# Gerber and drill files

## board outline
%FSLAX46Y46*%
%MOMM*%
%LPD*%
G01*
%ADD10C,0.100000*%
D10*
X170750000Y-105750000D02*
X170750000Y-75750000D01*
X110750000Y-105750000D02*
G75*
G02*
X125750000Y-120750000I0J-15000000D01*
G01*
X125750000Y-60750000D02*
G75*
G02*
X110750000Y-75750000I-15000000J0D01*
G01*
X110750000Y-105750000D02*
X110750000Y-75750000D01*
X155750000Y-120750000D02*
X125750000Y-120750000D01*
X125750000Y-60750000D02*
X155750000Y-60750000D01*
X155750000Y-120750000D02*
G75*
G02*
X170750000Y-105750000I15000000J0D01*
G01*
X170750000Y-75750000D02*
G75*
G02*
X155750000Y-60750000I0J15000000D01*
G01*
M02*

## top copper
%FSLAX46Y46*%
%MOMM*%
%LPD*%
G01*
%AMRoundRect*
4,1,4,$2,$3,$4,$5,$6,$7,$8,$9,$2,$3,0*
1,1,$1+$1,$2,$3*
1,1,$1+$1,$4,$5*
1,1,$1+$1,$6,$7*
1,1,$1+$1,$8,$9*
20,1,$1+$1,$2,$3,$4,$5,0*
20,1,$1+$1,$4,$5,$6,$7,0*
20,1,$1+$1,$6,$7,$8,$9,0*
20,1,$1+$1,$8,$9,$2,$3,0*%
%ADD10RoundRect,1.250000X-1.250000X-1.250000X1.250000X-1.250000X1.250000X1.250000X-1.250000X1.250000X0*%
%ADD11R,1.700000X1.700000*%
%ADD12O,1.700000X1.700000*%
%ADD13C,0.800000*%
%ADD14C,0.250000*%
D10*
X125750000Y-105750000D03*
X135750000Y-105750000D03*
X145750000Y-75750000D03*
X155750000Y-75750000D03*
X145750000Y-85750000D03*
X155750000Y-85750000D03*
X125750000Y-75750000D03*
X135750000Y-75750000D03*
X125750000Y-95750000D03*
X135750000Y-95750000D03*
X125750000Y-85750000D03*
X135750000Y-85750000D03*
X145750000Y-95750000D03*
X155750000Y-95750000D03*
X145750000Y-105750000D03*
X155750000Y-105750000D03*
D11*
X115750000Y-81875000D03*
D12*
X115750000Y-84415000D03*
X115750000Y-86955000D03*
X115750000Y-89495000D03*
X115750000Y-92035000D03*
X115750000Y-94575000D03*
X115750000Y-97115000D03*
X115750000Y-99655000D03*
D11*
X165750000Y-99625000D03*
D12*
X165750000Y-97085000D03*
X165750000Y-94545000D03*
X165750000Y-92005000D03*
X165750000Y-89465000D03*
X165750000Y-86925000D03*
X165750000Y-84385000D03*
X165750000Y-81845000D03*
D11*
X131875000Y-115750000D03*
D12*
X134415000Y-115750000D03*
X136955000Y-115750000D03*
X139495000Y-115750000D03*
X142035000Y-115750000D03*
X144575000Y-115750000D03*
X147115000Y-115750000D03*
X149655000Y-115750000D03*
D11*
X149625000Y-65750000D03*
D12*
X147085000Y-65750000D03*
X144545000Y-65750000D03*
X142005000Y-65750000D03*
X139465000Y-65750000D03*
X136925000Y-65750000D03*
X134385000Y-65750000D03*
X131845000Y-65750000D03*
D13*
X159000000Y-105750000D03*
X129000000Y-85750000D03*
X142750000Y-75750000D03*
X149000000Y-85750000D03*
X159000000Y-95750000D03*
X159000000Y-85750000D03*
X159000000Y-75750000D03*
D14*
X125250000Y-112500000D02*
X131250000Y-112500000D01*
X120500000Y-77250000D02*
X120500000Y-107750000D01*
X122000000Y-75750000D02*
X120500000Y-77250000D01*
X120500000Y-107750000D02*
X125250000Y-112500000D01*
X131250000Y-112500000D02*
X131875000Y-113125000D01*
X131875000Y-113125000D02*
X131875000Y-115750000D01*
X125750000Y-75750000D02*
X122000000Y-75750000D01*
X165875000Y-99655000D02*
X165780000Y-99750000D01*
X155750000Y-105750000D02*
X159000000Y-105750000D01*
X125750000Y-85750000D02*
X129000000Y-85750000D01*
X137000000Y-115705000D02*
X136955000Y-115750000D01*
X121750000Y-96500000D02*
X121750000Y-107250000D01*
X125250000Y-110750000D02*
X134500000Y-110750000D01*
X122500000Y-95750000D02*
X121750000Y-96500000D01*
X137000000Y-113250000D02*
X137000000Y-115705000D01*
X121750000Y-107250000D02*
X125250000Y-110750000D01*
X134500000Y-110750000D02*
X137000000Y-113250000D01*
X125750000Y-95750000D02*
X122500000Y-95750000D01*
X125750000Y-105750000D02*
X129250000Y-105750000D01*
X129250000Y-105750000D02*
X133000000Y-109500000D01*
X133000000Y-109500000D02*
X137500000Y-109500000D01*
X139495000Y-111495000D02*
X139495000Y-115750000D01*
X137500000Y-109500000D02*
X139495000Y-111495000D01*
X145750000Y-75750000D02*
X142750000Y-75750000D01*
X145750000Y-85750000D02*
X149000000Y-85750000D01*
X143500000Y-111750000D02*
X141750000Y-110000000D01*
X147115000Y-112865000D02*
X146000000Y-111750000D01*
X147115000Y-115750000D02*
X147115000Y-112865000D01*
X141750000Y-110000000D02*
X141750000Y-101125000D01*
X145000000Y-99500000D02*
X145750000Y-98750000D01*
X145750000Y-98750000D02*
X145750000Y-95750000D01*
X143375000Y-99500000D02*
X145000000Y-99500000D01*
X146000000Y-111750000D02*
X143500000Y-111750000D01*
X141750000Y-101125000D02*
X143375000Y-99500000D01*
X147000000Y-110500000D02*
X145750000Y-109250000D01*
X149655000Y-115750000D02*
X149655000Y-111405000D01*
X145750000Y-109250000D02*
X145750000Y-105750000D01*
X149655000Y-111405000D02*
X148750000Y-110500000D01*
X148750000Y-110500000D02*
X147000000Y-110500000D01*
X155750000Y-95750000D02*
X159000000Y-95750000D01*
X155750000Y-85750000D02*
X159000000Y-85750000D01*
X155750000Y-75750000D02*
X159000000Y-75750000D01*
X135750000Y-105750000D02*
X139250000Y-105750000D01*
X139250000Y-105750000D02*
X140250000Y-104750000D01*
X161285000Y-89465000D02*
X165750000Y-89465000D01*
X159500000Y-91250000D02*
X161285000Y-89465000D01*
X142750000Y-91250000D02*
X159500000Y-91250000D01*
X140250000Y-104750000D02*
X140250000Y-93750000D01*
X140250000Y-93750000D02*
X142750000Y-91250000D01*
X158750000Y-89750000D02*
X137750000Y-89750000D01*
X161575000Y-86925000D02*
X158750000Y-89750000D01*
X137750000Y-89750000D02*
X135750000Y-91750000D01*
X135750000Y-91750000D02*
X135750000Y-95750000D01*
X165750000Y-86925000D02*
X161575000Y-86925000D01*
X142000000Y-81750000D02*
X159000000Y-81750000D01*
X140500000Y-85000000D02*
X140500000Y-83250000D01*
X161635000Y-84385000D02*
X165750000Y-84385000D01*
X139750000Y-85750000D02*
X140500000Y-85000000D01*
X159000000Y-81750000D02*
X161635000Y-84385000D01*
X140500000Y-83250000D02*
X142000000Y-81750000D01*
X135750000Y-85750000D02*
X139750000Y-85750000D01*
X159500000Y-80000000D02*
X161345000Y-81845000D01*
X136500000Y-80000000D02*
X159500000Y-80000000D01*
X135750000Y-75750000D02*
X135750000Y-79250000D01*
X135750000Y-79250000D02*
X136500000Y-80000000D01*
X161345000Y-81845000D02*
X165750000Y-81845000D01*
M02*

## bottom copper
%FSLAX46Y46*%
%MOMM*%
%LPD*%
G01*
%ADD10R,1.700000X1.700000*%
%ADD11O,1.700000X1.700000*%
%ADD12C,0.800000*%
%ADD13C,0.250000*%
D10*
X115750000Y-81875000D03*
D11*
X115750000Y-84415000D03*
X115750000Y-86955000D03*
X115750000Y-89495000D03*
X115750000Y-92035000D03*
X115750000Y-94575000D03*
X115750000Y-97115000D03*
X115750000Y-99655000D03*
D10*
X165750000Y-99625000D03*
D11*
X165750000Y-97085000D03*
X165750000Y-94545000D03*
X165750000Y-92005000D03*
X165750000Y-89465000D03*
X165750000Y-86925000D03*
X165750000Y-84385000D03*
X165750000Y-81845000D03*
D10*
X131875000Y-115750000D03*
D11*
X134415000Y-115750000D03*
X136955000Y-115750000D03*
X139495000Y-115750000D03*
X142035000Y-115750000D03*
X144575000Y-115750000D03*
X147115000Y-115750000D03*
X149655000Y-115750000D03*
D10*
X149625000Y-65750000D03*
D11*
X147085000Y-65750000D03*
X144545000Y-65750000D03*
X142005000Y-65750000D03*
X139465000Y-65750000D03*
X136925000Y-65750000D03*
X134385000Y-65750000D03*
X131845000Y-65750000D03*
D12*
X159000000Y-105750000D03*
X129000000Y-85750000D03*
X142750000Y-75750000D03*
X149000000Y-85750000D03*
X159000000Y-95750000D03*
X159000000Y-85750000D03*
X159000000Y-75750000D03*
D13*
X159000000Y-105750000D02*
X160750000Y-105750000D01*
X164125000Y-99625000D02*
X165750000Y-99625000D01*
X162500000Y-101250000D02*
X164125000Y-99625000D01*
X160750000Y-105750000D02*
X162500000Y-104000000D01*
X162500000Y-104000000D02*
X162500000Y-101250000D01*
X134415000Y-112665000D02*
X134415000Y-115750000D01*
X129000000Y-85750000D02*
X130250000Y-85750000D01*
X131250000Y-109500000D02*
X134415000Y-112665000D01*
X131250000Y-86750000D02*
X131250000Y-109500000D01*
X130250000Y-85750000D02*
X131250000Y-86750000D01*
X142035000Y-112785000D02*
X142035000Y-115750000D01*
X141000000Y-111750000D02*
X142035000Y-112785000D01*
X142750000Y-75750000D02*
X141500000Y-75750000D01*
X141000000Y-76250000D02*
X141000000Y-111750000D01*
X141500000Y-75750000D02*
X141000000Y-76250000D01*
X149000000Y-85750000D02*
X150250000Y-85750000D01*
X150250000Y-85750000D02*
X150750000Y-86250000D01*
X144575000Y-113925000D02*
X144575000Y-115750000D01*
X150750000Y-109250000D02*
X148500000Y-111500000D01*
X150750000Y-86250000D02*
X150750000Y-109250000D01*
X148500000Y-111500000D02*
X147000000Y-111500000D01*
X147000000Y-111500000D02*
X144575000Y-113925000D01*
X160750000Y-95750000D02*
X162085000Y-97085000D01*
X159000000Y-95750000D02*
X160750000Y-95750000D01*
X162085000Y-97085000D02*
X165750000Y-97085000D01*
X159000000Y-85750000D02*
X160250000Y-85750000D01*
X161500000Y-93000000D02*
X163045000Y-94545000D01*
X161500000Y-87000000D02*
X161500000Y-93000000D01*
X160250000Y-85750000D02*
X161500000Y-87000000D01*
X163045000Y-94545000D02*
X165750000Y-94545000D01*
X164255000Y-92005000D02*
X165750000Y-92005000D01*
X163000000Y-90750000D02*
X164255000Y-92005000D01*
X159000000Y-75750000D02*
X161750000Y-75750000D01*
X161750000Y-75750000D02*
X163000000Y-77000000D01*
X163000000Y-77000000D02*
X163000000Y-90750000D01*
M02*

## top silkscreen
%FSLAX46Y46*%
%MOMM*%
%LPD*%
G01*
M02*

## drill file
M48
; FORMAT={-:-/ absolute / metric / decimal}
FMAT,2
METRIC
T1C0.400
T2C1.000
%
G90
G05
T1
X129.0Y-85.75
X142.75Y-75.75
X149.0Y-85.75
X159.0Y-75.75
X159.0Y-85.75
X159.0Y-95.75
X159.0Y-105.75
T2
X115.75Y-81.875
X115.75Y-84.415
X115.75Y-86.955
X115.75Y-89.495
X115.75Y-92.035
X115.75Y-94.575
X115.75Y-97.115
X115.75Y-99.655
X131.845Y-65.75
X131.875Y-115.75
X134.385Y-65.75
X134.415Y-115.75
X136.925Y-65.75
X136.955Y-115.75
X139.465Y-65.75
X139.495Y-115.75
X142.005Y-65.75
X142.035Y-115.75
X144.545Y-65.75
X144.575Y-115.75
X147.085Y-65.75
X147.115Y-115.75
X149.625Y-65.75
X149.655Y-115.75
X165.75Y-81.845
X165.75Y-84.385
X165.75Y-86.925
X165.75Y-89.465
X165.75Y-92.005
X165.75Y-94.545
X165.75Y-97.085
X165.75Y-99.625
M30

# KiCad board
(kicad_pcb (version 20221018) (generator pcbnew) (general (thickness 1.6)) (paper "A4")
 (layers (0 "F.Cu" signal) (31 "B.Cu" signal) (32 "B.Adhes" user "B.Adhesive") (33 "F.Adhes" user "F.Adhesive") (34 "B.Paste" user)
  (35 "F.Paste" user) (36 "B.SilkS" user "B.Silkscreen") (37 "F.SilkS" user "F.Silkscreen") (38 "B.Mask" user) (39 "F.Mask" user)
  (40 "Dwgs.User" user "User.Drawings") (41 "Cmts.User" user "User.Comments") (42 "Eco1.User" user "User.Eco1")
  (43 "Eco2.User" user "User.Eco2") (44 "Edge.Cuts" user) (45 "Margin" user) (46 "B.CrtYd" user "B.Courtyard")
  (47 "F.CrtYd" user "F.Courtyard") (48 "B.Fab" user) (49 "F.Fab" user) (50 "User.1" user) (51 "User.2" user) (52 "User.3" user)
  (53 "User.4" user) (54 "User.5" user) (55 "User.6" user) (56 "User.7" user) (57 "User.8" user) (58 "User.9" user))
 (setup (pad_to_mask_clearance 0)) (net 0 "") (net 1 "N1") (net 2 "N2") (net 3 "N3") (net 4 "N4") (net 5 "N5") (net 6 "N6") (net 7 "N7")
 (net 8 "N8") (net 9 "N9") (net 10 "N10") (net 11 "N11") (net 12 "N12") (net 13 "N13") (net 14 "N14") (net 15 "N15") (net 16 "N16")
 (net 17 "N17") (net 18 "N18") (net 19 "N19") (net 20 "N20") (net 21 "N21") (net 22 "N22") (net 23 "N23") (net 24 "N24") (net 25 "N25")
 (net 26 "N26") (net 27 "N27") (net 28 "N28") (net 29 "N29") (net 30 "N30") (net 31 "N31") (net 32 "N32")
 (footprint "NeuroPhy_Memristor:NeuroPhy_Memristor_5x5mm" (layer "F.Cu") (at 130.75 105.75)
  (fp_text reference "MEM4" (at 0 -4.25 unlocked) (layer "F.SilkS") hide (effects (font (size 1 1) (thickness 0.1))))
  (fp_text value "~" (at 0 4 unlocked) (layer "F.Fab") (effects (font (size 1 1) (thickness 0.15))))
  (pad "1" smd roundrect (at -5 0) (size 5 5) (layers "F.Cu" "F.Mask") (roundrect_rratio 0.25) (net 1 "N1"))
  (pad "2" smd roundrect (at 5 0) (size 5 5) (layers "F.Cu" "F.Mask") (roundrect_rratio 0.25) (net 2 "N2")))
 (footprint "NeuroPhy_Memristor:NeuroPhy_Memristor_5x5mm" (layer "F.Cu") (at 150.75 75.75)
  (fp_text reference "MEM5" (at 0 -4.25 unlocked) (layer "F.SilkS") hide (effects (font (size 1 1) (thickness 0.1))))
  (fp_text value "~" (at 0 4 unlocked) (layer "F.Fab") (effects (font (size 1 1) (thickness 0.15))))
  (pad "1" smd roundrect (at -5 0) (size 5 5) (layers "F.Cu" "F.Mask") (roundrect_rratio 0.25) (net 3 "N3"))
  (pad "2" smd roundrect (at 5 0) (size 5 5) (layers "F.Cu" "F.Mask") (roundrect_rratio 0.25) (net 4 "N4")))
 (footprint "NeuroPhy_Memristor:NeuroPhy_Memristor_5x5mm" (layer "F.Cu") (at 150.75 85.75)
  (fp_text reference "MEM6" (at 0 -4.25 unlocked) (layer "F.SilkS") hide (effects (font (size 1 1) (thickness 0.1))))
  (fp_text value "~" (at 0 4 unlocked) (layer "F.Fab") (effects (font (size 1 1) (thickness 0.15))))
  (pad "1" smd roundrect (at -5 0) (size 5 5) (layers "F.Cu" "F.Mask") (roundrect_rratio 0.25) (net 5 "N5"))
  (pad "2" smd roundrect (at 5 0) (size 5 5) (layers "F.Cu" "F.Mask") (roundrect_rratio 0.25) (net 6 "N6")))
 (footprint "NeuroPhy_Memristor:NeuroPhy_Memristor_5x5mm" (layer "F.Cu") (at 130.75 75.75)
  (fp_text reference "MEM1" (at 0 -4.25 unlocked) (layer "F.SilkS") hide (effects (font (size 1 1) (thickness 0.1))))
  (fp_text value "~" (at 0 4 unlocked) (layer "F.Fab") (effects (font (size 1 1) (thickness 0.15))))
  (pad "1" smd roundrect (at -5 0) (size 5 5) (layers "F.Cu" "F.Mask") (roundrect_rratio 0.25) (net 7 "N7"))
  (pad "2" smd roundrect (at 5 0) (size 5 5) (layers "F.Cu" "F.Mask") (roundrect_rratio 0.25) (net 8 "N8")))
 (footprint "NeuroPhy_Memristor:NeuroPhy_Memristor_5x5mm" (layer "F.Cu") (at 130.75 95.75)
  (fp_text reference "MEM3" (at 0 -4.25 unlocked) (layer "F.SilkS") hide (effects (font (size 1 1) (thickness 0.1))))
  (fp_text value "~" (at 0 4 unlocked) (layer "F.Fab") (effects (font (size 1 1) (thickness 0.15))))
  (pad "1" smd roundrect (at -5 0) (size 5 5) (layers "F.Cu" "F.Mask") (roundrect_rratio 0.25) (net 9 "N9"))
  (pad "2" smd roundrect (at 5 0) (size 5 5) (layers "F.Cu" "F.Mask") (roundrect_rratio 0.25) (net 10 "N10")))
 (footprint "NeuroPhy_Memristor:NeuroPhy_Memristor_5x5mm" (layer "F.Cu") (at 130.75 85.75)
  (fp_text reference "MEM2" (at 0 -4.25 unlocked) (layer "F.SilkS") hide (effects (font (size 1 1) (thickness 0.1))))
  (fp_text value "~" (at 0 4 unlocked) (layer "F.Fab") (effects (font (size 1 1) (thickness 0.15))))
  (pad "1" smd roundrect (at -5 0) (size 5 5) (layers "F.Cu" "F.Mask") (roundrect_rratio 0.25) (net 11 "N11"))
  (pad "2" smd roundrect (at 5 0) (size 5 5) (layers "F.Cu" "F.Mask") (roundrect_rratio 0.25) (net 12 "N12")))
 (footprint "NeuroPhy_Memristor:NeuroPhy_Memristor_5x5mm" (layer "F.Cu") (at 150.75 95.75)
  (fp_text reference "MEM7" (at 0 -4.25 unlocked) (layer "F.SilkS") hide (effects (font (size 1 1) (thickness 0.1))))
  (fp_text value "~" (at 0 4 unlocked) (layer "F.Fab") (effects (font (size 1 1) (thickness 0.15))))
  (pad "1" smd roundrect (at -5 0) (size 5 5) (layers "F.Cu" "F.Mask") (roundrect_rratio 0.25) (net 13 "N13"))
  (pad "2" smd roundrect (at 5 0) (size 5 5) (layers "F.Cu" "F.Mask") (roundrect_rratio 0.25) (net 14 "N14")))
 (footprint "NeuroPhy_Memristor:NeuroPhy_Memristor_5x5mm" (layer "F.Cu") (at 150.75 105.75)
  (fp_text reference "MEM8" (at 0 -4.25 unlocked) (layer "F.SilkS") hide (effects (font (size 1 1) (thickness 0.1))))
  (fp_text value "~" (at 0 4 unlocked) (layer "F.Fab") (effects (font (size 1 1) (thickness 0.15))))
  (pad "1" smd roundrect (at -5 0) (size 5 5) (layers "F.Cu" "F.Mask") (roundrect_rratio 0.25) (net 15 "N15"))
  (pad "2" smd roundrect (at 5 0) (size 5 5) (layers "F.Cu" "F.Mask") (roundrect_rratio 0.25) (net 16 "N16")))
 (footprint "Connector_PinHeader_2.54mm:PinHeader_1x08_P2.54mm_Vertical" (layer "B.Cu") (at 115.75 81.875 180)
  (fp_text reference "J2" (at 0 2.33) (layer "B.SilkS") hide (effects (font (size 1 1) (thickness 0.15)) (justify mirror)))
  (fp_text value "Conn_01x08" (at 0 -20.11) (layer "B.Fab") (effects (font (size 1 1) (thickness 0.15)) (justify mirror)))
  (pad "1" thru_hole rect (at 0 0 180) (size 1.7 1.7) (drill 1) (layers "*.Cu" "*.Mask") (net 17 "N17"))
  (pad "2" thru_hole oval (at 0 -2.54 180) (size 1.7 1.7) (drill 1) (layers "*.Cu" "*.Mask") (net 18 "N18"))
  (pad "3" thru_hole oval (at 0 -5.08 180) (size 1.7 1.7) (drill 1) (layers "*.Cu" "*.Mask") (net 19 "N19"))
  (pad "4" thru_hole oval (at 0 -7.62 180) (size 1.7 1.7) (drill 1) (layers "*.Cu" "*.Mask") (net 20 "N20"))
  (pad "5" thru_hole oval (at 0 -10.16 180) (size 1.7 1.7) (drill 1) (layers "*.Cu" "*.Mask") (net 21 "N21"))
  (pad "6" thru_hole oval (at 0 -12.7 180) (size 1.7 1.7) (drill 1) (layers "*.Cu" "*.Mask") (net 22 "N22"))
  (pad "7" thru_hole oval (at 0 -15.24 180) (size 1.7 1.7) (drill 1) (layers "*.Cu" "*.Mask") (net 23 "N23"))
  (pad "8" thru_hole oval (at 0 -17.78 180) (size 1.7 1.7) (drill 1) (layers "*.Cu" "*.Mask") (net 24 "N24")))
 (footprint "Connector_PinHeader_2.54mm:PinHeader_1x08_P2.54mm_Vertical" (layer "B.Cu") (at 165.75 99.625)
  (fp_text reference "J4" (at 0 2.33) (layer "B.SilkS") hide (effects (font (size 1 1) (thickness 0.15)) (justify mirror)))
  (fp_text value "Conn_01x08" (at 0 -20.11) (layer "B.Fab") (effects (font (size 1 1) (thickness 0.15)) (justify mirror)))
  (pad "1" thru_hole rect (at 0 0) (size 1.7 1.7) (drill 1) (layers "*.Cu" "*.Mask") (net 16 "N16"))
  (pad "2" thru_hole oval (at 0 -2.54) (size 1.7 1.7) (drill 1) (layers "*.Cu" "*.Mask") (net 14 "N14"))
  (pad "3" thru_hole oval (at 0 -5.08) (size 1.7 1.7) (drill 1) (layers "*.Cu" "*.Mask") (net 6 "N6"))
  (pad "4" thru_hole oval (at 0 -7.62) (size 1.7 1.7) (drill 1) (layers "*.Cu" "*.Mask") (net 4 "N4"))
  (pad "5" thru_hole oval (at 0 -10.16) (size 1.7 1.7) (drill 1) (layers "*.Cu" "*.Mask") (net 2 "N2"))
  (pad "6" thru_hole oval (at 0 -12.7) (size 1.7 1.7) (drill 1) (layers "*.Cu" "*.Mask") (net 10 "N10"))
  (pad "7" thru_hole oval (at 0 -15.24) (size 1.7 1.7) (drill 1) (layers "*.Cu" "*.Mask") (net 12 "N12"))
  (pad "8" thru_hole oval (at 0 -17.78) (size 1.7 1.7) (drill 1) (layers "*.Cu" "*.Mask") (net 8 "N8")))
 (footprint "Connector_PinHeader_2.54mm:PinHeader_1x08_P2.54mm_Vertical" (layer "B.Cu") (at 131.875 115.75 -90)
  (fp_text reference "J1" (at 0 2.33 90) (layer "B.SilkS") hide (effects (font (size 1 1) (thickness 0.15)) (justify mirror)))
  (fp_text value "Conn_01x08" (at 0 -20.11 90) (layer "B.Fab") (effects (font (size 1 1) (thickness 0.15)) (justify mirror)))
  (pad "1" thru_hole rect (at 0 0 270) (size 1.7 1.7) (drill 1) (layers "*.Cu" "*.Mask") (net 7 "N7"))
  (pad "2" thru_hole oval (at 0 -2.54 270) (size 1.7 1.7) (drill 1) (layers "*.Cu" "*.Mask") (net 11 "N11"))
  (pad "3" thru_hole oval (at 0 -5.08 270) (size 1.7 1.7) (drill 1) (layers "*.Cu" "*.Mask") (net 9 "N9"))
  (pad "4" thru_hole oval (at 0 -7.62 270) (size 1.7 1.7) (drill 1) (layers "*.Cu" "*.Mask") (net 1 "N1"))
  (pad "5" thru_hole oval (at 0 -10.16 270) (size 1.7 1.7) (drill 1) (layers "*.Cu" "*.Mask") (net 3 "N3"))
  (pad "6" thru_hole oval (at 0 -12.7 270) (size 1.7 1.7) (drill 1) (layers "*.Cu" "*.Mask") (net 5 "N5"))
  (pad "7" thru_hole oval (at 0 -15.24 270) (size 1.7 1.7) (drill 1) (layers "*.Cu" "*.Mask") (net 13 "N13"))
  (pad "8" thru_hole oval (at 0 -17.78 270) (size 1.7 1.7) (drill 1) (layers "*.Cu" "*.Mask") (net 15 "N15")))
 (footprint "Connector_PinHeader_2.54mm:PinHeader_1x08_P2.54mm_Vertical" (layer "B.Cu") (at 149.625 65.75 90)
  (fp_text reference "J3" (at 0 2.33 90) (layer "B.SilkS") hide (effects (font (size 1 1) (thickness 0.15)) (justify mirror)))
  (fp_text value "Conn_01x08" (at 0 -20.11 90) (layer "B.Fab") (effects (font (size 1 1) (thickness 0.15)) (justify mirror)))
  (pad "1" thru_hole rect (at 0 0 90) (size 1.7 1.7) (drill 1) (layers "*.Cu" "*.Mask") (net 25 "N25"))
  (pad "2" thru_hole oval (at 0 -2.54 90) (size 1.7 1.7) (drill 1) (layers "*.Cu" "*.Mask") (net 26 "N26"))
  (pad "3" thru_hole oval (at 0 -5.08 90) (size 1.7 1.7) (drill 1) (layers "*.Cu" "*.Mask") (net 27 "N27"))
  (pad "4" thru_hole oval (at 0 -7.62 90) (size 1.7 1.7) (drill 1) (layers "*.Cu" "*.Mask") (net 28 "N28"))
  (pad "5" thru_hole oval (at 0 -10.16 90) (size 1.7 1.7) (drill 1) (layers "*.Cu" "*.Mask") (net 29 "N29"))
  (pad "6" thru_hole oval (at 0 -12.7 90) (size 1.7 1.7) (drill 1) (layers "*.Cu" "*.Mask") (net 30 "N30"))
  (pad "7" thru_hole oval (at 0 -15.24 90) (size 1.7 1.7) (drill 1) (layers "*.Cu" "*.Mask") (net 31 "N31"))
  (pad "8" thru_hole oval (at 0 -17.78 90) (size 1.7 1.7) (drill 1) (layers "*.Cu" "*.Mask") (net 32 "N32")))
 (gr_line (start 170.75 105.75) (end 170.75 75.75) (stroke (width 0.1) (type default)) (layer "Edge.Cuts"))
 (gr_arc (start 110.75 105.75) (mid 121.356602 110.143398) (end 125.75 120.75) (stroke (width 0.1) (type default)) (layer "Edge.Cuts"))
 (gr_arc (start 125.75 60.75) (mid 121.356602 71.356602) (end 110.75 75.75) (stroke (width 0.1) (type default)) (layer "Edge.Cuts"))
 (gr_line (start 110.75 105.75) (end 110.75 75.75) (stroke (width 0.1) (type default)) (layer "Edge.Cuts"))
 (gr_line (start 155.75 120.75) (end 125.75 120.75) (stroke (width 0.1) (type default)) (layer "Edge.Cuts"))
 (gr_line (start 125.75 60.75) (end 155.75 60.75) (stroke (width 0.1) (type default)) (layer "Edge.Cuts"))
 (gr_arc (start 155.75 120.75) (mid 160.143398 110.143398) (end 170.75 105.75) (stroke (width 0.1) (type default)) (layer "Edge.Cuts"))
 (gr_arc (start 170.75 75.75) (mid 160.143398 71.356602) (end 155.75 60.75) (stroke (width 0.1) (type default)) (layer "Edge.Cuts"))
 (segment (start 125.25 112.5) (end 131.25 112.5) (width 0.25) (layer "F.Cu") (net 7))
 (segment (start 120.5 77.25) (end 120.5 107.75) (width 0.25) (layer "F.Cu") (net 7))
 (segment (start 122 75.75) (end 120.5 77.25) (width 0.25) (layer "F.Cu") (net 7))
 (segment (start 120.5 107.75) (end 125.25 112.5) (width 0.25) (layer "F.Cu") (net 7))
 (segment (start 131.25 112.5) (end 131.875 113.125) (width 0.25) (layer "F.Cu") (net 7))
 (segment (start 131.875 113.125) (end 131.875 115.75) (width 0.25) (layer "F.Cu") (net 7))
 (segment (start 125.75 75.75) (end 122 75.75) (width 0.25) (layer "F.Cu") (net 7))
 (segment (start 165.875 99.655) (end 165.78 99.75) (width 0.25) (layer "F.Cu") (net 16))
 (segment (start 155.75 105.75) (end 159 105.75) (width 0.25) (layer "F.Cu") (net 16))
 (via (at 159 105.75) (size 0.8) (drill 0.4) (layers "F.Cu" "B.Cu") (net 16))
 (segment (start 159 105.75) (end 160.75 105.75) (width 0.25) (layer "B.Cu") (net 16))
 (segment (start 164.125 99.625) (end 165.75 99.625) (width 0.25) (layer "B.Cu") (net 16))
 (segment (start 162.5 101.25) (end 164.125 99.625) (width 0.25) (layer "B.Cu") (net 16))
 (segment (start 160.75 105.75) (end 162.5 104) (width 0.25) (layer "B.Cu") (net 16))
 (segment (start 162.5 104) (end 162.5 101.25) (width 0.25) (layer "B.Cu") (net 16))
 (segment (start 125.75 85.75) (end 129 85.75) (width 0.25) (layer "F.Cu") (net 11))
 (via (at 129 85.75) (size 0.8) (drill 0.4) (layers "F.Cu" "B.Cu") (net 11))
 (segment (start 134.415 112.665) (end 134.415 115.75) (width 0.25) (layer "B.Cu") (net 11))
 (segment (start 129 85.75) (end 130.25 85.75) (width 0.25) (layer "B.Cu") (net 11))
 (segment (start 131.25 109.5) (end 134.415 112.665) (width 0.25) (layer "B.Cu") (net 11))
 (segment (start 131.25 86.75) (end 131.25 109.5) (width 0.25) (layer "B.Cu") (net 11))
 (segment (start 130.25 85.75) (end 131.25 86.75) (width 0.25) (layer "B.Cu") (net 11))
 (segment (start 137 115.705) (end 136.955 115.75) (width 0.25) (layer "F.Cu") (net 9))
 (segment (start 121.75 96.5) (end 121.75 107.25) (width 0.25) (layer "F.Cu") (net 9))
 (segment (start 125.25 110.75) (end 134.5 110.75) (width 0.25) (layer "F.Cu") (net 9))
 (segment (start 122.5 95.75) (end 121.75 96.5) (width 0.25) (layer "F.Cu") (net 9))
 (segment (start 137 113.25) (end 137 115.705) (width 0.25) (layer "F.Cu") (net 9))
 (segment (start 121.75 107.25) (end 125.25 110.75) (width 0.25) (layer "F.Cu") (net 9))
 (segment (start 134.5 110.75) (end 137 113.25) (width 0.25) (layer "F.Cu") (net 9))
 (segment (start 125.75 95.75) (end 122.5 95.75) (width 0.25) (layer "F.Cu") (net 9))
 (segment (start 125.75 105.75) (end 129.25 105.75) (width 0.25) (layer "F.Cu") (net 1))
 (segment (start 129.25 105.75) (end 133 109.5) (width 0.25) (layer "F.Cu") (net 1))
 (segment (start 133 109.5) (end 137.5 109.5) (width 0.25) (layer "F.Cu") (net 1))
 (segment (start 139.495 111.495) (end 139.495 115.75) (width 0.25) (layer "F.Cu") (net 1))
 (segment (start 137.5 109.5) (end 139.495 111.495) (width 0.25) (layer "F.Cu") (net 1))
 (segment (start 145.75 75.75) (end 142.75 75.75) (width 0.25) (layer "F.Cu") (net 3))
 (via (at 142.75 75.75) (size 0.8) (drill 0.4) (layers "F.Cu" "B.Cu") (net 3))
 (segment (start 142.035 112.785) (end 142.035 115.75) (width 0.25) (layer "B.Cu") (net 3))
 (segment (start 141 111.75) (end 142.035 112.785) (width 0.25) (layer "B.Cu") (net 3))
 (segment (start 142.75 75.75) (end 141.5 75.75) (width 0.25) (layer "B.Cu") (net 3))
 (segment (start 141 76.25) (end 141 111.75) (width 0.25) (layer "B.Cu") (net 3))
 (segment (start 141.5 75.75) (end 141 76.25) (width 0.25) (layer "B.Cu") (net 3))
 (segment (start 145.75 85.75) (end 149 85.75) (width 0.25) (layer "F.Cu") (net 5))
 (via (at 149 85.75) (size 0.8) (drill 0.4) (layers "F.Cu" "B.Cu") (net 5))
 (segment (start 149 85.75) (end 150.25 85.75) (width 0.25) (layer "B.Cu") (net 5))
 (segment (start 150.25 85.75) (end 150.75 86.25) (width 0.25) (layer "B.Cu") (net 5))
 (segment (start 144.575 113.925) (end 144.575 115.75) (width 0.25) (layer "B.Cu") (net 5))
 (segment (start 150.75 109.25) (end 148.5 111.5) (width 0.25) (layer "B.Cu") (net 5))
 (segment (start 150.75 86.25) (end 150.75 109.25) (width 0.25) (layer "B.Cu") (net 5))
 (segment (start 148.5 111.5) (end 147 111.5) (width 0.25) (layer "B.Cu") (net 5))
 (segment (start 147 111.5) (end 144.575 113.925) (width 0.25) (layer "B.Cu") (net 5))
 (segment (start 143.5 111.75) (end 141.75 110) (width 0.25) (layer "F.Cu") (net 13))
 (segment (start 147.115 112.865) (end 146 111.75) (width 0.25) (layer "F.Cu") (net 13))
 (segment (start 147.115 115.75) (end 147.115 112.865) (width 0.25) (layer "F.Cu") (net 13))
 (segment (start 141.75 110) (end 141.75 101.125) (width 0.25) (layer "F.Cu") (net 13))
 (segment (start 145 99.5) (end 145.75 98.75) (width 0.25) (layer "F.Cu") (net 13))
 (segment (start 145.75 98.75) (end 145.75 95.75) (width 0.25) (layer "F.Cu") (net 13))
 (segment (start 143.375 99.5) (end 145 99.5) (width 0.25) (layer "F.Cu") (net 13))
 (segment (start 146 111.75) (end 143.5 111.75) (width 0.25) (layer "F.Cu") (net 13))
 (segment (start 141.75 101.125) (end 143.375 99.5) (width 0.25) (layer "F.Cu") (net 13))
 (segment (start 147 110.5) (end 145.75 109.25) (width 0.25) (layer "F.Cu") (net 15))
 (segment (start 149.655 115.75) (end 149.655 111.405) (width 0.25) (layer "F.Cu") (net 15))
 (segment (start 145.75 109.25) (end 145.75 105.75) (width 0.25) (layer "F.Cu") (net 15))
 (segment (start 149.655 111.405) (end 148.75 110.5) (width 0.25) (layer "F.Cu") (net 15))
 (segment (start 148.75 110.5) (end 147 110.5) (width 0.25) (layer "F.Cu") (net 15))
 (segment (start 155.75 95.75) (end 159 95.75) (width 0.25) (layer "F.Cu") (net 14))
 (via (at 159 95.75) (size 0.8) (drill 0.4) (layers "F.Cu" "B.Cu") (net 14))
 (segment (start 160.75 95.75) (end 162.085 97.085) (width 0.25) (layer "B.Cu") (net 14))
 (segment (start 159 95.75) (end 160.75 95.75) (width 0.25) (layer "B.Cu") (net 14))
 (segment (start 162.085 97.085) (end 165.75 97.085) (width 0.25) (layer "B.Cu") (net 14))
 (segment (start 155.75 85.75) (end 159 85.75) (width 0.25) (layer "F.Cu") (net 6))
 (via (at 159 85.75) (size 0.8) (drill 0.4) (layers "F.Cu" "B.Cu") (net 6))
 (segment (start 159 85.75) (end 160.25 85.75) (width 0.25) (layer "B.Cu") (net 6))
 (segment (start 161.5 93) (end 163.045 94.545) (width 0.25) (layer "B.Cu") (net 6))
 (segment (start 161.5 87) (end 161.5 93) (width 0.25) (layer "B.Cu") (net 6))
 (segment (start 160.25 85.75) (end 161.5 87) (width 0.25) (layer "B.Cu") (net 6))
 (segment (start 163.045 94.545) (end 165.75 94.545) (width 0.25) (layer "B.Cu") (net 6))
 (segment (start 155.75 75.75) (end 159 75.75) (width 0.25) (layer "F.Cu") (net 4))
 (via (at 159 75.75) (size 0.8) (drill 0.4) (layers "F.Cu" "B.Cu") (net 4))
 (segment (start 164.255 92.005) (end 165.75 92.005) (width 0.25) (layer "B.Cu") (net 4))
 (segment (start 163 90.75) (end 164.255 92.005) (width 0.25) (layer "B.Cu") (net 4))
 (segment (start 159 75.75) (end 161.75 75.75) (width 0.25) (layer "B.Cu") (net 4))
 (segment (start 161.75 75.75) (end 163 77) (width 0.25) (layer "B.Cu") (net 4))
 (segment (start 163 77) (end 163 90.75) (width 0.25) (layer "B.Cu") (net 4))
 (segment (start 135.75 105.75) (end 139.25 105.75) (width 0.25) (layer "F.Cu") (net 2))
 (segment (start 139.25 105.75) (end 140.25 104.75) (width 0.25) (layer "F.Cu") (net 2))
 (segment (start 161.285 89.465) (end 165.75 89.465) (width 0.25) (layer "F.Cu") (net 2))
 (segment (start 159.5 91.25) (end 161.285 89.465) (width 0.25) (layer "F.Cu") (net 2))
 (segment (start 142.75 91.25) (end 159.5 91.25) (width 0.25) (layer "F.Cu") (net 2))
 (segment (start 140.25 104.75) (end 140.25 93.75) (width 0.25) (layer "F.Cu") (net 2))
 (segment (start 140.25 93.75) (end 142.75 91.25) (width 0.25) (layer "F.Cu") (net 2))
 (segment (start 158.75 89.75) (end 137.75 89.75) (width 0.25) (layer "F.Cu") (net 10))
 (segment (start 161.575 86.925) (end 158.75 89.75) (width 0.25) (layer "F.Cu") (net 10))
 (segment (start 137.75 89.75) (end 135.75 91.75) (width 0.25) (layer "F.Cu") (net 10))
 (segment (start 135.75 91.75) (end 135.75 95.75) (width 0.25) (layer "F.Cu") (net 10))
 (segment (start 165.75 86.925) (end 161.575 86.925) (width 0.25) (layer "F.Cu") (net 10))
 (segment (start 142 81.75) (end 159 81.75) (width 0.25) (layer "F.Cu") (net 12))
 (segment (start 140.5 85) (end 140.5 83.25) (width 0.25) (layer "F.Cu") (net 12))
 (segment (start 161.635 84.385) (end 165.75 84.385) (width 0.25) (layer "F.Cu") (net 12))
 (segment (start 139.75 85.75) (end 140.5 85) (width 0.25) (layer "F.Cu") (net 12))
 (segment (start 159 81.75) (end 161.635 84.385) (width 0.25) (layer "F.Cu") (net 12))
 (segment (start 140.5 83.25) (end 142 81.75) (width 0.25) (layer "F.Cu") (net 12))
 (segment (start 135.75 85.75) (end 139.75 85.75) (width 0.25) (layer "F.Cu") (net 12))
 (segment (start 159.5 80) (end 161.345 81.845) (width 0.25) (layer "F.Cu") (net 8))
 (segment (start 136.5 80) (end 159.5 80) (width 0.25) (layer "F.Cu") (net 8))
 (segment (start 135.75 75.75) (end 135.75 79.25) (width 0.25) (layer "F.Cu") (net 8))
 (segment (start 135.75 79.25) (end 136.5 80) (width 0.25) (layer "F.Cu") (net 8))
 (segment (start 161.345 81.845) (end 165.75 81.845) (width 0.25) (layer "F.Cu") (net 8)))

